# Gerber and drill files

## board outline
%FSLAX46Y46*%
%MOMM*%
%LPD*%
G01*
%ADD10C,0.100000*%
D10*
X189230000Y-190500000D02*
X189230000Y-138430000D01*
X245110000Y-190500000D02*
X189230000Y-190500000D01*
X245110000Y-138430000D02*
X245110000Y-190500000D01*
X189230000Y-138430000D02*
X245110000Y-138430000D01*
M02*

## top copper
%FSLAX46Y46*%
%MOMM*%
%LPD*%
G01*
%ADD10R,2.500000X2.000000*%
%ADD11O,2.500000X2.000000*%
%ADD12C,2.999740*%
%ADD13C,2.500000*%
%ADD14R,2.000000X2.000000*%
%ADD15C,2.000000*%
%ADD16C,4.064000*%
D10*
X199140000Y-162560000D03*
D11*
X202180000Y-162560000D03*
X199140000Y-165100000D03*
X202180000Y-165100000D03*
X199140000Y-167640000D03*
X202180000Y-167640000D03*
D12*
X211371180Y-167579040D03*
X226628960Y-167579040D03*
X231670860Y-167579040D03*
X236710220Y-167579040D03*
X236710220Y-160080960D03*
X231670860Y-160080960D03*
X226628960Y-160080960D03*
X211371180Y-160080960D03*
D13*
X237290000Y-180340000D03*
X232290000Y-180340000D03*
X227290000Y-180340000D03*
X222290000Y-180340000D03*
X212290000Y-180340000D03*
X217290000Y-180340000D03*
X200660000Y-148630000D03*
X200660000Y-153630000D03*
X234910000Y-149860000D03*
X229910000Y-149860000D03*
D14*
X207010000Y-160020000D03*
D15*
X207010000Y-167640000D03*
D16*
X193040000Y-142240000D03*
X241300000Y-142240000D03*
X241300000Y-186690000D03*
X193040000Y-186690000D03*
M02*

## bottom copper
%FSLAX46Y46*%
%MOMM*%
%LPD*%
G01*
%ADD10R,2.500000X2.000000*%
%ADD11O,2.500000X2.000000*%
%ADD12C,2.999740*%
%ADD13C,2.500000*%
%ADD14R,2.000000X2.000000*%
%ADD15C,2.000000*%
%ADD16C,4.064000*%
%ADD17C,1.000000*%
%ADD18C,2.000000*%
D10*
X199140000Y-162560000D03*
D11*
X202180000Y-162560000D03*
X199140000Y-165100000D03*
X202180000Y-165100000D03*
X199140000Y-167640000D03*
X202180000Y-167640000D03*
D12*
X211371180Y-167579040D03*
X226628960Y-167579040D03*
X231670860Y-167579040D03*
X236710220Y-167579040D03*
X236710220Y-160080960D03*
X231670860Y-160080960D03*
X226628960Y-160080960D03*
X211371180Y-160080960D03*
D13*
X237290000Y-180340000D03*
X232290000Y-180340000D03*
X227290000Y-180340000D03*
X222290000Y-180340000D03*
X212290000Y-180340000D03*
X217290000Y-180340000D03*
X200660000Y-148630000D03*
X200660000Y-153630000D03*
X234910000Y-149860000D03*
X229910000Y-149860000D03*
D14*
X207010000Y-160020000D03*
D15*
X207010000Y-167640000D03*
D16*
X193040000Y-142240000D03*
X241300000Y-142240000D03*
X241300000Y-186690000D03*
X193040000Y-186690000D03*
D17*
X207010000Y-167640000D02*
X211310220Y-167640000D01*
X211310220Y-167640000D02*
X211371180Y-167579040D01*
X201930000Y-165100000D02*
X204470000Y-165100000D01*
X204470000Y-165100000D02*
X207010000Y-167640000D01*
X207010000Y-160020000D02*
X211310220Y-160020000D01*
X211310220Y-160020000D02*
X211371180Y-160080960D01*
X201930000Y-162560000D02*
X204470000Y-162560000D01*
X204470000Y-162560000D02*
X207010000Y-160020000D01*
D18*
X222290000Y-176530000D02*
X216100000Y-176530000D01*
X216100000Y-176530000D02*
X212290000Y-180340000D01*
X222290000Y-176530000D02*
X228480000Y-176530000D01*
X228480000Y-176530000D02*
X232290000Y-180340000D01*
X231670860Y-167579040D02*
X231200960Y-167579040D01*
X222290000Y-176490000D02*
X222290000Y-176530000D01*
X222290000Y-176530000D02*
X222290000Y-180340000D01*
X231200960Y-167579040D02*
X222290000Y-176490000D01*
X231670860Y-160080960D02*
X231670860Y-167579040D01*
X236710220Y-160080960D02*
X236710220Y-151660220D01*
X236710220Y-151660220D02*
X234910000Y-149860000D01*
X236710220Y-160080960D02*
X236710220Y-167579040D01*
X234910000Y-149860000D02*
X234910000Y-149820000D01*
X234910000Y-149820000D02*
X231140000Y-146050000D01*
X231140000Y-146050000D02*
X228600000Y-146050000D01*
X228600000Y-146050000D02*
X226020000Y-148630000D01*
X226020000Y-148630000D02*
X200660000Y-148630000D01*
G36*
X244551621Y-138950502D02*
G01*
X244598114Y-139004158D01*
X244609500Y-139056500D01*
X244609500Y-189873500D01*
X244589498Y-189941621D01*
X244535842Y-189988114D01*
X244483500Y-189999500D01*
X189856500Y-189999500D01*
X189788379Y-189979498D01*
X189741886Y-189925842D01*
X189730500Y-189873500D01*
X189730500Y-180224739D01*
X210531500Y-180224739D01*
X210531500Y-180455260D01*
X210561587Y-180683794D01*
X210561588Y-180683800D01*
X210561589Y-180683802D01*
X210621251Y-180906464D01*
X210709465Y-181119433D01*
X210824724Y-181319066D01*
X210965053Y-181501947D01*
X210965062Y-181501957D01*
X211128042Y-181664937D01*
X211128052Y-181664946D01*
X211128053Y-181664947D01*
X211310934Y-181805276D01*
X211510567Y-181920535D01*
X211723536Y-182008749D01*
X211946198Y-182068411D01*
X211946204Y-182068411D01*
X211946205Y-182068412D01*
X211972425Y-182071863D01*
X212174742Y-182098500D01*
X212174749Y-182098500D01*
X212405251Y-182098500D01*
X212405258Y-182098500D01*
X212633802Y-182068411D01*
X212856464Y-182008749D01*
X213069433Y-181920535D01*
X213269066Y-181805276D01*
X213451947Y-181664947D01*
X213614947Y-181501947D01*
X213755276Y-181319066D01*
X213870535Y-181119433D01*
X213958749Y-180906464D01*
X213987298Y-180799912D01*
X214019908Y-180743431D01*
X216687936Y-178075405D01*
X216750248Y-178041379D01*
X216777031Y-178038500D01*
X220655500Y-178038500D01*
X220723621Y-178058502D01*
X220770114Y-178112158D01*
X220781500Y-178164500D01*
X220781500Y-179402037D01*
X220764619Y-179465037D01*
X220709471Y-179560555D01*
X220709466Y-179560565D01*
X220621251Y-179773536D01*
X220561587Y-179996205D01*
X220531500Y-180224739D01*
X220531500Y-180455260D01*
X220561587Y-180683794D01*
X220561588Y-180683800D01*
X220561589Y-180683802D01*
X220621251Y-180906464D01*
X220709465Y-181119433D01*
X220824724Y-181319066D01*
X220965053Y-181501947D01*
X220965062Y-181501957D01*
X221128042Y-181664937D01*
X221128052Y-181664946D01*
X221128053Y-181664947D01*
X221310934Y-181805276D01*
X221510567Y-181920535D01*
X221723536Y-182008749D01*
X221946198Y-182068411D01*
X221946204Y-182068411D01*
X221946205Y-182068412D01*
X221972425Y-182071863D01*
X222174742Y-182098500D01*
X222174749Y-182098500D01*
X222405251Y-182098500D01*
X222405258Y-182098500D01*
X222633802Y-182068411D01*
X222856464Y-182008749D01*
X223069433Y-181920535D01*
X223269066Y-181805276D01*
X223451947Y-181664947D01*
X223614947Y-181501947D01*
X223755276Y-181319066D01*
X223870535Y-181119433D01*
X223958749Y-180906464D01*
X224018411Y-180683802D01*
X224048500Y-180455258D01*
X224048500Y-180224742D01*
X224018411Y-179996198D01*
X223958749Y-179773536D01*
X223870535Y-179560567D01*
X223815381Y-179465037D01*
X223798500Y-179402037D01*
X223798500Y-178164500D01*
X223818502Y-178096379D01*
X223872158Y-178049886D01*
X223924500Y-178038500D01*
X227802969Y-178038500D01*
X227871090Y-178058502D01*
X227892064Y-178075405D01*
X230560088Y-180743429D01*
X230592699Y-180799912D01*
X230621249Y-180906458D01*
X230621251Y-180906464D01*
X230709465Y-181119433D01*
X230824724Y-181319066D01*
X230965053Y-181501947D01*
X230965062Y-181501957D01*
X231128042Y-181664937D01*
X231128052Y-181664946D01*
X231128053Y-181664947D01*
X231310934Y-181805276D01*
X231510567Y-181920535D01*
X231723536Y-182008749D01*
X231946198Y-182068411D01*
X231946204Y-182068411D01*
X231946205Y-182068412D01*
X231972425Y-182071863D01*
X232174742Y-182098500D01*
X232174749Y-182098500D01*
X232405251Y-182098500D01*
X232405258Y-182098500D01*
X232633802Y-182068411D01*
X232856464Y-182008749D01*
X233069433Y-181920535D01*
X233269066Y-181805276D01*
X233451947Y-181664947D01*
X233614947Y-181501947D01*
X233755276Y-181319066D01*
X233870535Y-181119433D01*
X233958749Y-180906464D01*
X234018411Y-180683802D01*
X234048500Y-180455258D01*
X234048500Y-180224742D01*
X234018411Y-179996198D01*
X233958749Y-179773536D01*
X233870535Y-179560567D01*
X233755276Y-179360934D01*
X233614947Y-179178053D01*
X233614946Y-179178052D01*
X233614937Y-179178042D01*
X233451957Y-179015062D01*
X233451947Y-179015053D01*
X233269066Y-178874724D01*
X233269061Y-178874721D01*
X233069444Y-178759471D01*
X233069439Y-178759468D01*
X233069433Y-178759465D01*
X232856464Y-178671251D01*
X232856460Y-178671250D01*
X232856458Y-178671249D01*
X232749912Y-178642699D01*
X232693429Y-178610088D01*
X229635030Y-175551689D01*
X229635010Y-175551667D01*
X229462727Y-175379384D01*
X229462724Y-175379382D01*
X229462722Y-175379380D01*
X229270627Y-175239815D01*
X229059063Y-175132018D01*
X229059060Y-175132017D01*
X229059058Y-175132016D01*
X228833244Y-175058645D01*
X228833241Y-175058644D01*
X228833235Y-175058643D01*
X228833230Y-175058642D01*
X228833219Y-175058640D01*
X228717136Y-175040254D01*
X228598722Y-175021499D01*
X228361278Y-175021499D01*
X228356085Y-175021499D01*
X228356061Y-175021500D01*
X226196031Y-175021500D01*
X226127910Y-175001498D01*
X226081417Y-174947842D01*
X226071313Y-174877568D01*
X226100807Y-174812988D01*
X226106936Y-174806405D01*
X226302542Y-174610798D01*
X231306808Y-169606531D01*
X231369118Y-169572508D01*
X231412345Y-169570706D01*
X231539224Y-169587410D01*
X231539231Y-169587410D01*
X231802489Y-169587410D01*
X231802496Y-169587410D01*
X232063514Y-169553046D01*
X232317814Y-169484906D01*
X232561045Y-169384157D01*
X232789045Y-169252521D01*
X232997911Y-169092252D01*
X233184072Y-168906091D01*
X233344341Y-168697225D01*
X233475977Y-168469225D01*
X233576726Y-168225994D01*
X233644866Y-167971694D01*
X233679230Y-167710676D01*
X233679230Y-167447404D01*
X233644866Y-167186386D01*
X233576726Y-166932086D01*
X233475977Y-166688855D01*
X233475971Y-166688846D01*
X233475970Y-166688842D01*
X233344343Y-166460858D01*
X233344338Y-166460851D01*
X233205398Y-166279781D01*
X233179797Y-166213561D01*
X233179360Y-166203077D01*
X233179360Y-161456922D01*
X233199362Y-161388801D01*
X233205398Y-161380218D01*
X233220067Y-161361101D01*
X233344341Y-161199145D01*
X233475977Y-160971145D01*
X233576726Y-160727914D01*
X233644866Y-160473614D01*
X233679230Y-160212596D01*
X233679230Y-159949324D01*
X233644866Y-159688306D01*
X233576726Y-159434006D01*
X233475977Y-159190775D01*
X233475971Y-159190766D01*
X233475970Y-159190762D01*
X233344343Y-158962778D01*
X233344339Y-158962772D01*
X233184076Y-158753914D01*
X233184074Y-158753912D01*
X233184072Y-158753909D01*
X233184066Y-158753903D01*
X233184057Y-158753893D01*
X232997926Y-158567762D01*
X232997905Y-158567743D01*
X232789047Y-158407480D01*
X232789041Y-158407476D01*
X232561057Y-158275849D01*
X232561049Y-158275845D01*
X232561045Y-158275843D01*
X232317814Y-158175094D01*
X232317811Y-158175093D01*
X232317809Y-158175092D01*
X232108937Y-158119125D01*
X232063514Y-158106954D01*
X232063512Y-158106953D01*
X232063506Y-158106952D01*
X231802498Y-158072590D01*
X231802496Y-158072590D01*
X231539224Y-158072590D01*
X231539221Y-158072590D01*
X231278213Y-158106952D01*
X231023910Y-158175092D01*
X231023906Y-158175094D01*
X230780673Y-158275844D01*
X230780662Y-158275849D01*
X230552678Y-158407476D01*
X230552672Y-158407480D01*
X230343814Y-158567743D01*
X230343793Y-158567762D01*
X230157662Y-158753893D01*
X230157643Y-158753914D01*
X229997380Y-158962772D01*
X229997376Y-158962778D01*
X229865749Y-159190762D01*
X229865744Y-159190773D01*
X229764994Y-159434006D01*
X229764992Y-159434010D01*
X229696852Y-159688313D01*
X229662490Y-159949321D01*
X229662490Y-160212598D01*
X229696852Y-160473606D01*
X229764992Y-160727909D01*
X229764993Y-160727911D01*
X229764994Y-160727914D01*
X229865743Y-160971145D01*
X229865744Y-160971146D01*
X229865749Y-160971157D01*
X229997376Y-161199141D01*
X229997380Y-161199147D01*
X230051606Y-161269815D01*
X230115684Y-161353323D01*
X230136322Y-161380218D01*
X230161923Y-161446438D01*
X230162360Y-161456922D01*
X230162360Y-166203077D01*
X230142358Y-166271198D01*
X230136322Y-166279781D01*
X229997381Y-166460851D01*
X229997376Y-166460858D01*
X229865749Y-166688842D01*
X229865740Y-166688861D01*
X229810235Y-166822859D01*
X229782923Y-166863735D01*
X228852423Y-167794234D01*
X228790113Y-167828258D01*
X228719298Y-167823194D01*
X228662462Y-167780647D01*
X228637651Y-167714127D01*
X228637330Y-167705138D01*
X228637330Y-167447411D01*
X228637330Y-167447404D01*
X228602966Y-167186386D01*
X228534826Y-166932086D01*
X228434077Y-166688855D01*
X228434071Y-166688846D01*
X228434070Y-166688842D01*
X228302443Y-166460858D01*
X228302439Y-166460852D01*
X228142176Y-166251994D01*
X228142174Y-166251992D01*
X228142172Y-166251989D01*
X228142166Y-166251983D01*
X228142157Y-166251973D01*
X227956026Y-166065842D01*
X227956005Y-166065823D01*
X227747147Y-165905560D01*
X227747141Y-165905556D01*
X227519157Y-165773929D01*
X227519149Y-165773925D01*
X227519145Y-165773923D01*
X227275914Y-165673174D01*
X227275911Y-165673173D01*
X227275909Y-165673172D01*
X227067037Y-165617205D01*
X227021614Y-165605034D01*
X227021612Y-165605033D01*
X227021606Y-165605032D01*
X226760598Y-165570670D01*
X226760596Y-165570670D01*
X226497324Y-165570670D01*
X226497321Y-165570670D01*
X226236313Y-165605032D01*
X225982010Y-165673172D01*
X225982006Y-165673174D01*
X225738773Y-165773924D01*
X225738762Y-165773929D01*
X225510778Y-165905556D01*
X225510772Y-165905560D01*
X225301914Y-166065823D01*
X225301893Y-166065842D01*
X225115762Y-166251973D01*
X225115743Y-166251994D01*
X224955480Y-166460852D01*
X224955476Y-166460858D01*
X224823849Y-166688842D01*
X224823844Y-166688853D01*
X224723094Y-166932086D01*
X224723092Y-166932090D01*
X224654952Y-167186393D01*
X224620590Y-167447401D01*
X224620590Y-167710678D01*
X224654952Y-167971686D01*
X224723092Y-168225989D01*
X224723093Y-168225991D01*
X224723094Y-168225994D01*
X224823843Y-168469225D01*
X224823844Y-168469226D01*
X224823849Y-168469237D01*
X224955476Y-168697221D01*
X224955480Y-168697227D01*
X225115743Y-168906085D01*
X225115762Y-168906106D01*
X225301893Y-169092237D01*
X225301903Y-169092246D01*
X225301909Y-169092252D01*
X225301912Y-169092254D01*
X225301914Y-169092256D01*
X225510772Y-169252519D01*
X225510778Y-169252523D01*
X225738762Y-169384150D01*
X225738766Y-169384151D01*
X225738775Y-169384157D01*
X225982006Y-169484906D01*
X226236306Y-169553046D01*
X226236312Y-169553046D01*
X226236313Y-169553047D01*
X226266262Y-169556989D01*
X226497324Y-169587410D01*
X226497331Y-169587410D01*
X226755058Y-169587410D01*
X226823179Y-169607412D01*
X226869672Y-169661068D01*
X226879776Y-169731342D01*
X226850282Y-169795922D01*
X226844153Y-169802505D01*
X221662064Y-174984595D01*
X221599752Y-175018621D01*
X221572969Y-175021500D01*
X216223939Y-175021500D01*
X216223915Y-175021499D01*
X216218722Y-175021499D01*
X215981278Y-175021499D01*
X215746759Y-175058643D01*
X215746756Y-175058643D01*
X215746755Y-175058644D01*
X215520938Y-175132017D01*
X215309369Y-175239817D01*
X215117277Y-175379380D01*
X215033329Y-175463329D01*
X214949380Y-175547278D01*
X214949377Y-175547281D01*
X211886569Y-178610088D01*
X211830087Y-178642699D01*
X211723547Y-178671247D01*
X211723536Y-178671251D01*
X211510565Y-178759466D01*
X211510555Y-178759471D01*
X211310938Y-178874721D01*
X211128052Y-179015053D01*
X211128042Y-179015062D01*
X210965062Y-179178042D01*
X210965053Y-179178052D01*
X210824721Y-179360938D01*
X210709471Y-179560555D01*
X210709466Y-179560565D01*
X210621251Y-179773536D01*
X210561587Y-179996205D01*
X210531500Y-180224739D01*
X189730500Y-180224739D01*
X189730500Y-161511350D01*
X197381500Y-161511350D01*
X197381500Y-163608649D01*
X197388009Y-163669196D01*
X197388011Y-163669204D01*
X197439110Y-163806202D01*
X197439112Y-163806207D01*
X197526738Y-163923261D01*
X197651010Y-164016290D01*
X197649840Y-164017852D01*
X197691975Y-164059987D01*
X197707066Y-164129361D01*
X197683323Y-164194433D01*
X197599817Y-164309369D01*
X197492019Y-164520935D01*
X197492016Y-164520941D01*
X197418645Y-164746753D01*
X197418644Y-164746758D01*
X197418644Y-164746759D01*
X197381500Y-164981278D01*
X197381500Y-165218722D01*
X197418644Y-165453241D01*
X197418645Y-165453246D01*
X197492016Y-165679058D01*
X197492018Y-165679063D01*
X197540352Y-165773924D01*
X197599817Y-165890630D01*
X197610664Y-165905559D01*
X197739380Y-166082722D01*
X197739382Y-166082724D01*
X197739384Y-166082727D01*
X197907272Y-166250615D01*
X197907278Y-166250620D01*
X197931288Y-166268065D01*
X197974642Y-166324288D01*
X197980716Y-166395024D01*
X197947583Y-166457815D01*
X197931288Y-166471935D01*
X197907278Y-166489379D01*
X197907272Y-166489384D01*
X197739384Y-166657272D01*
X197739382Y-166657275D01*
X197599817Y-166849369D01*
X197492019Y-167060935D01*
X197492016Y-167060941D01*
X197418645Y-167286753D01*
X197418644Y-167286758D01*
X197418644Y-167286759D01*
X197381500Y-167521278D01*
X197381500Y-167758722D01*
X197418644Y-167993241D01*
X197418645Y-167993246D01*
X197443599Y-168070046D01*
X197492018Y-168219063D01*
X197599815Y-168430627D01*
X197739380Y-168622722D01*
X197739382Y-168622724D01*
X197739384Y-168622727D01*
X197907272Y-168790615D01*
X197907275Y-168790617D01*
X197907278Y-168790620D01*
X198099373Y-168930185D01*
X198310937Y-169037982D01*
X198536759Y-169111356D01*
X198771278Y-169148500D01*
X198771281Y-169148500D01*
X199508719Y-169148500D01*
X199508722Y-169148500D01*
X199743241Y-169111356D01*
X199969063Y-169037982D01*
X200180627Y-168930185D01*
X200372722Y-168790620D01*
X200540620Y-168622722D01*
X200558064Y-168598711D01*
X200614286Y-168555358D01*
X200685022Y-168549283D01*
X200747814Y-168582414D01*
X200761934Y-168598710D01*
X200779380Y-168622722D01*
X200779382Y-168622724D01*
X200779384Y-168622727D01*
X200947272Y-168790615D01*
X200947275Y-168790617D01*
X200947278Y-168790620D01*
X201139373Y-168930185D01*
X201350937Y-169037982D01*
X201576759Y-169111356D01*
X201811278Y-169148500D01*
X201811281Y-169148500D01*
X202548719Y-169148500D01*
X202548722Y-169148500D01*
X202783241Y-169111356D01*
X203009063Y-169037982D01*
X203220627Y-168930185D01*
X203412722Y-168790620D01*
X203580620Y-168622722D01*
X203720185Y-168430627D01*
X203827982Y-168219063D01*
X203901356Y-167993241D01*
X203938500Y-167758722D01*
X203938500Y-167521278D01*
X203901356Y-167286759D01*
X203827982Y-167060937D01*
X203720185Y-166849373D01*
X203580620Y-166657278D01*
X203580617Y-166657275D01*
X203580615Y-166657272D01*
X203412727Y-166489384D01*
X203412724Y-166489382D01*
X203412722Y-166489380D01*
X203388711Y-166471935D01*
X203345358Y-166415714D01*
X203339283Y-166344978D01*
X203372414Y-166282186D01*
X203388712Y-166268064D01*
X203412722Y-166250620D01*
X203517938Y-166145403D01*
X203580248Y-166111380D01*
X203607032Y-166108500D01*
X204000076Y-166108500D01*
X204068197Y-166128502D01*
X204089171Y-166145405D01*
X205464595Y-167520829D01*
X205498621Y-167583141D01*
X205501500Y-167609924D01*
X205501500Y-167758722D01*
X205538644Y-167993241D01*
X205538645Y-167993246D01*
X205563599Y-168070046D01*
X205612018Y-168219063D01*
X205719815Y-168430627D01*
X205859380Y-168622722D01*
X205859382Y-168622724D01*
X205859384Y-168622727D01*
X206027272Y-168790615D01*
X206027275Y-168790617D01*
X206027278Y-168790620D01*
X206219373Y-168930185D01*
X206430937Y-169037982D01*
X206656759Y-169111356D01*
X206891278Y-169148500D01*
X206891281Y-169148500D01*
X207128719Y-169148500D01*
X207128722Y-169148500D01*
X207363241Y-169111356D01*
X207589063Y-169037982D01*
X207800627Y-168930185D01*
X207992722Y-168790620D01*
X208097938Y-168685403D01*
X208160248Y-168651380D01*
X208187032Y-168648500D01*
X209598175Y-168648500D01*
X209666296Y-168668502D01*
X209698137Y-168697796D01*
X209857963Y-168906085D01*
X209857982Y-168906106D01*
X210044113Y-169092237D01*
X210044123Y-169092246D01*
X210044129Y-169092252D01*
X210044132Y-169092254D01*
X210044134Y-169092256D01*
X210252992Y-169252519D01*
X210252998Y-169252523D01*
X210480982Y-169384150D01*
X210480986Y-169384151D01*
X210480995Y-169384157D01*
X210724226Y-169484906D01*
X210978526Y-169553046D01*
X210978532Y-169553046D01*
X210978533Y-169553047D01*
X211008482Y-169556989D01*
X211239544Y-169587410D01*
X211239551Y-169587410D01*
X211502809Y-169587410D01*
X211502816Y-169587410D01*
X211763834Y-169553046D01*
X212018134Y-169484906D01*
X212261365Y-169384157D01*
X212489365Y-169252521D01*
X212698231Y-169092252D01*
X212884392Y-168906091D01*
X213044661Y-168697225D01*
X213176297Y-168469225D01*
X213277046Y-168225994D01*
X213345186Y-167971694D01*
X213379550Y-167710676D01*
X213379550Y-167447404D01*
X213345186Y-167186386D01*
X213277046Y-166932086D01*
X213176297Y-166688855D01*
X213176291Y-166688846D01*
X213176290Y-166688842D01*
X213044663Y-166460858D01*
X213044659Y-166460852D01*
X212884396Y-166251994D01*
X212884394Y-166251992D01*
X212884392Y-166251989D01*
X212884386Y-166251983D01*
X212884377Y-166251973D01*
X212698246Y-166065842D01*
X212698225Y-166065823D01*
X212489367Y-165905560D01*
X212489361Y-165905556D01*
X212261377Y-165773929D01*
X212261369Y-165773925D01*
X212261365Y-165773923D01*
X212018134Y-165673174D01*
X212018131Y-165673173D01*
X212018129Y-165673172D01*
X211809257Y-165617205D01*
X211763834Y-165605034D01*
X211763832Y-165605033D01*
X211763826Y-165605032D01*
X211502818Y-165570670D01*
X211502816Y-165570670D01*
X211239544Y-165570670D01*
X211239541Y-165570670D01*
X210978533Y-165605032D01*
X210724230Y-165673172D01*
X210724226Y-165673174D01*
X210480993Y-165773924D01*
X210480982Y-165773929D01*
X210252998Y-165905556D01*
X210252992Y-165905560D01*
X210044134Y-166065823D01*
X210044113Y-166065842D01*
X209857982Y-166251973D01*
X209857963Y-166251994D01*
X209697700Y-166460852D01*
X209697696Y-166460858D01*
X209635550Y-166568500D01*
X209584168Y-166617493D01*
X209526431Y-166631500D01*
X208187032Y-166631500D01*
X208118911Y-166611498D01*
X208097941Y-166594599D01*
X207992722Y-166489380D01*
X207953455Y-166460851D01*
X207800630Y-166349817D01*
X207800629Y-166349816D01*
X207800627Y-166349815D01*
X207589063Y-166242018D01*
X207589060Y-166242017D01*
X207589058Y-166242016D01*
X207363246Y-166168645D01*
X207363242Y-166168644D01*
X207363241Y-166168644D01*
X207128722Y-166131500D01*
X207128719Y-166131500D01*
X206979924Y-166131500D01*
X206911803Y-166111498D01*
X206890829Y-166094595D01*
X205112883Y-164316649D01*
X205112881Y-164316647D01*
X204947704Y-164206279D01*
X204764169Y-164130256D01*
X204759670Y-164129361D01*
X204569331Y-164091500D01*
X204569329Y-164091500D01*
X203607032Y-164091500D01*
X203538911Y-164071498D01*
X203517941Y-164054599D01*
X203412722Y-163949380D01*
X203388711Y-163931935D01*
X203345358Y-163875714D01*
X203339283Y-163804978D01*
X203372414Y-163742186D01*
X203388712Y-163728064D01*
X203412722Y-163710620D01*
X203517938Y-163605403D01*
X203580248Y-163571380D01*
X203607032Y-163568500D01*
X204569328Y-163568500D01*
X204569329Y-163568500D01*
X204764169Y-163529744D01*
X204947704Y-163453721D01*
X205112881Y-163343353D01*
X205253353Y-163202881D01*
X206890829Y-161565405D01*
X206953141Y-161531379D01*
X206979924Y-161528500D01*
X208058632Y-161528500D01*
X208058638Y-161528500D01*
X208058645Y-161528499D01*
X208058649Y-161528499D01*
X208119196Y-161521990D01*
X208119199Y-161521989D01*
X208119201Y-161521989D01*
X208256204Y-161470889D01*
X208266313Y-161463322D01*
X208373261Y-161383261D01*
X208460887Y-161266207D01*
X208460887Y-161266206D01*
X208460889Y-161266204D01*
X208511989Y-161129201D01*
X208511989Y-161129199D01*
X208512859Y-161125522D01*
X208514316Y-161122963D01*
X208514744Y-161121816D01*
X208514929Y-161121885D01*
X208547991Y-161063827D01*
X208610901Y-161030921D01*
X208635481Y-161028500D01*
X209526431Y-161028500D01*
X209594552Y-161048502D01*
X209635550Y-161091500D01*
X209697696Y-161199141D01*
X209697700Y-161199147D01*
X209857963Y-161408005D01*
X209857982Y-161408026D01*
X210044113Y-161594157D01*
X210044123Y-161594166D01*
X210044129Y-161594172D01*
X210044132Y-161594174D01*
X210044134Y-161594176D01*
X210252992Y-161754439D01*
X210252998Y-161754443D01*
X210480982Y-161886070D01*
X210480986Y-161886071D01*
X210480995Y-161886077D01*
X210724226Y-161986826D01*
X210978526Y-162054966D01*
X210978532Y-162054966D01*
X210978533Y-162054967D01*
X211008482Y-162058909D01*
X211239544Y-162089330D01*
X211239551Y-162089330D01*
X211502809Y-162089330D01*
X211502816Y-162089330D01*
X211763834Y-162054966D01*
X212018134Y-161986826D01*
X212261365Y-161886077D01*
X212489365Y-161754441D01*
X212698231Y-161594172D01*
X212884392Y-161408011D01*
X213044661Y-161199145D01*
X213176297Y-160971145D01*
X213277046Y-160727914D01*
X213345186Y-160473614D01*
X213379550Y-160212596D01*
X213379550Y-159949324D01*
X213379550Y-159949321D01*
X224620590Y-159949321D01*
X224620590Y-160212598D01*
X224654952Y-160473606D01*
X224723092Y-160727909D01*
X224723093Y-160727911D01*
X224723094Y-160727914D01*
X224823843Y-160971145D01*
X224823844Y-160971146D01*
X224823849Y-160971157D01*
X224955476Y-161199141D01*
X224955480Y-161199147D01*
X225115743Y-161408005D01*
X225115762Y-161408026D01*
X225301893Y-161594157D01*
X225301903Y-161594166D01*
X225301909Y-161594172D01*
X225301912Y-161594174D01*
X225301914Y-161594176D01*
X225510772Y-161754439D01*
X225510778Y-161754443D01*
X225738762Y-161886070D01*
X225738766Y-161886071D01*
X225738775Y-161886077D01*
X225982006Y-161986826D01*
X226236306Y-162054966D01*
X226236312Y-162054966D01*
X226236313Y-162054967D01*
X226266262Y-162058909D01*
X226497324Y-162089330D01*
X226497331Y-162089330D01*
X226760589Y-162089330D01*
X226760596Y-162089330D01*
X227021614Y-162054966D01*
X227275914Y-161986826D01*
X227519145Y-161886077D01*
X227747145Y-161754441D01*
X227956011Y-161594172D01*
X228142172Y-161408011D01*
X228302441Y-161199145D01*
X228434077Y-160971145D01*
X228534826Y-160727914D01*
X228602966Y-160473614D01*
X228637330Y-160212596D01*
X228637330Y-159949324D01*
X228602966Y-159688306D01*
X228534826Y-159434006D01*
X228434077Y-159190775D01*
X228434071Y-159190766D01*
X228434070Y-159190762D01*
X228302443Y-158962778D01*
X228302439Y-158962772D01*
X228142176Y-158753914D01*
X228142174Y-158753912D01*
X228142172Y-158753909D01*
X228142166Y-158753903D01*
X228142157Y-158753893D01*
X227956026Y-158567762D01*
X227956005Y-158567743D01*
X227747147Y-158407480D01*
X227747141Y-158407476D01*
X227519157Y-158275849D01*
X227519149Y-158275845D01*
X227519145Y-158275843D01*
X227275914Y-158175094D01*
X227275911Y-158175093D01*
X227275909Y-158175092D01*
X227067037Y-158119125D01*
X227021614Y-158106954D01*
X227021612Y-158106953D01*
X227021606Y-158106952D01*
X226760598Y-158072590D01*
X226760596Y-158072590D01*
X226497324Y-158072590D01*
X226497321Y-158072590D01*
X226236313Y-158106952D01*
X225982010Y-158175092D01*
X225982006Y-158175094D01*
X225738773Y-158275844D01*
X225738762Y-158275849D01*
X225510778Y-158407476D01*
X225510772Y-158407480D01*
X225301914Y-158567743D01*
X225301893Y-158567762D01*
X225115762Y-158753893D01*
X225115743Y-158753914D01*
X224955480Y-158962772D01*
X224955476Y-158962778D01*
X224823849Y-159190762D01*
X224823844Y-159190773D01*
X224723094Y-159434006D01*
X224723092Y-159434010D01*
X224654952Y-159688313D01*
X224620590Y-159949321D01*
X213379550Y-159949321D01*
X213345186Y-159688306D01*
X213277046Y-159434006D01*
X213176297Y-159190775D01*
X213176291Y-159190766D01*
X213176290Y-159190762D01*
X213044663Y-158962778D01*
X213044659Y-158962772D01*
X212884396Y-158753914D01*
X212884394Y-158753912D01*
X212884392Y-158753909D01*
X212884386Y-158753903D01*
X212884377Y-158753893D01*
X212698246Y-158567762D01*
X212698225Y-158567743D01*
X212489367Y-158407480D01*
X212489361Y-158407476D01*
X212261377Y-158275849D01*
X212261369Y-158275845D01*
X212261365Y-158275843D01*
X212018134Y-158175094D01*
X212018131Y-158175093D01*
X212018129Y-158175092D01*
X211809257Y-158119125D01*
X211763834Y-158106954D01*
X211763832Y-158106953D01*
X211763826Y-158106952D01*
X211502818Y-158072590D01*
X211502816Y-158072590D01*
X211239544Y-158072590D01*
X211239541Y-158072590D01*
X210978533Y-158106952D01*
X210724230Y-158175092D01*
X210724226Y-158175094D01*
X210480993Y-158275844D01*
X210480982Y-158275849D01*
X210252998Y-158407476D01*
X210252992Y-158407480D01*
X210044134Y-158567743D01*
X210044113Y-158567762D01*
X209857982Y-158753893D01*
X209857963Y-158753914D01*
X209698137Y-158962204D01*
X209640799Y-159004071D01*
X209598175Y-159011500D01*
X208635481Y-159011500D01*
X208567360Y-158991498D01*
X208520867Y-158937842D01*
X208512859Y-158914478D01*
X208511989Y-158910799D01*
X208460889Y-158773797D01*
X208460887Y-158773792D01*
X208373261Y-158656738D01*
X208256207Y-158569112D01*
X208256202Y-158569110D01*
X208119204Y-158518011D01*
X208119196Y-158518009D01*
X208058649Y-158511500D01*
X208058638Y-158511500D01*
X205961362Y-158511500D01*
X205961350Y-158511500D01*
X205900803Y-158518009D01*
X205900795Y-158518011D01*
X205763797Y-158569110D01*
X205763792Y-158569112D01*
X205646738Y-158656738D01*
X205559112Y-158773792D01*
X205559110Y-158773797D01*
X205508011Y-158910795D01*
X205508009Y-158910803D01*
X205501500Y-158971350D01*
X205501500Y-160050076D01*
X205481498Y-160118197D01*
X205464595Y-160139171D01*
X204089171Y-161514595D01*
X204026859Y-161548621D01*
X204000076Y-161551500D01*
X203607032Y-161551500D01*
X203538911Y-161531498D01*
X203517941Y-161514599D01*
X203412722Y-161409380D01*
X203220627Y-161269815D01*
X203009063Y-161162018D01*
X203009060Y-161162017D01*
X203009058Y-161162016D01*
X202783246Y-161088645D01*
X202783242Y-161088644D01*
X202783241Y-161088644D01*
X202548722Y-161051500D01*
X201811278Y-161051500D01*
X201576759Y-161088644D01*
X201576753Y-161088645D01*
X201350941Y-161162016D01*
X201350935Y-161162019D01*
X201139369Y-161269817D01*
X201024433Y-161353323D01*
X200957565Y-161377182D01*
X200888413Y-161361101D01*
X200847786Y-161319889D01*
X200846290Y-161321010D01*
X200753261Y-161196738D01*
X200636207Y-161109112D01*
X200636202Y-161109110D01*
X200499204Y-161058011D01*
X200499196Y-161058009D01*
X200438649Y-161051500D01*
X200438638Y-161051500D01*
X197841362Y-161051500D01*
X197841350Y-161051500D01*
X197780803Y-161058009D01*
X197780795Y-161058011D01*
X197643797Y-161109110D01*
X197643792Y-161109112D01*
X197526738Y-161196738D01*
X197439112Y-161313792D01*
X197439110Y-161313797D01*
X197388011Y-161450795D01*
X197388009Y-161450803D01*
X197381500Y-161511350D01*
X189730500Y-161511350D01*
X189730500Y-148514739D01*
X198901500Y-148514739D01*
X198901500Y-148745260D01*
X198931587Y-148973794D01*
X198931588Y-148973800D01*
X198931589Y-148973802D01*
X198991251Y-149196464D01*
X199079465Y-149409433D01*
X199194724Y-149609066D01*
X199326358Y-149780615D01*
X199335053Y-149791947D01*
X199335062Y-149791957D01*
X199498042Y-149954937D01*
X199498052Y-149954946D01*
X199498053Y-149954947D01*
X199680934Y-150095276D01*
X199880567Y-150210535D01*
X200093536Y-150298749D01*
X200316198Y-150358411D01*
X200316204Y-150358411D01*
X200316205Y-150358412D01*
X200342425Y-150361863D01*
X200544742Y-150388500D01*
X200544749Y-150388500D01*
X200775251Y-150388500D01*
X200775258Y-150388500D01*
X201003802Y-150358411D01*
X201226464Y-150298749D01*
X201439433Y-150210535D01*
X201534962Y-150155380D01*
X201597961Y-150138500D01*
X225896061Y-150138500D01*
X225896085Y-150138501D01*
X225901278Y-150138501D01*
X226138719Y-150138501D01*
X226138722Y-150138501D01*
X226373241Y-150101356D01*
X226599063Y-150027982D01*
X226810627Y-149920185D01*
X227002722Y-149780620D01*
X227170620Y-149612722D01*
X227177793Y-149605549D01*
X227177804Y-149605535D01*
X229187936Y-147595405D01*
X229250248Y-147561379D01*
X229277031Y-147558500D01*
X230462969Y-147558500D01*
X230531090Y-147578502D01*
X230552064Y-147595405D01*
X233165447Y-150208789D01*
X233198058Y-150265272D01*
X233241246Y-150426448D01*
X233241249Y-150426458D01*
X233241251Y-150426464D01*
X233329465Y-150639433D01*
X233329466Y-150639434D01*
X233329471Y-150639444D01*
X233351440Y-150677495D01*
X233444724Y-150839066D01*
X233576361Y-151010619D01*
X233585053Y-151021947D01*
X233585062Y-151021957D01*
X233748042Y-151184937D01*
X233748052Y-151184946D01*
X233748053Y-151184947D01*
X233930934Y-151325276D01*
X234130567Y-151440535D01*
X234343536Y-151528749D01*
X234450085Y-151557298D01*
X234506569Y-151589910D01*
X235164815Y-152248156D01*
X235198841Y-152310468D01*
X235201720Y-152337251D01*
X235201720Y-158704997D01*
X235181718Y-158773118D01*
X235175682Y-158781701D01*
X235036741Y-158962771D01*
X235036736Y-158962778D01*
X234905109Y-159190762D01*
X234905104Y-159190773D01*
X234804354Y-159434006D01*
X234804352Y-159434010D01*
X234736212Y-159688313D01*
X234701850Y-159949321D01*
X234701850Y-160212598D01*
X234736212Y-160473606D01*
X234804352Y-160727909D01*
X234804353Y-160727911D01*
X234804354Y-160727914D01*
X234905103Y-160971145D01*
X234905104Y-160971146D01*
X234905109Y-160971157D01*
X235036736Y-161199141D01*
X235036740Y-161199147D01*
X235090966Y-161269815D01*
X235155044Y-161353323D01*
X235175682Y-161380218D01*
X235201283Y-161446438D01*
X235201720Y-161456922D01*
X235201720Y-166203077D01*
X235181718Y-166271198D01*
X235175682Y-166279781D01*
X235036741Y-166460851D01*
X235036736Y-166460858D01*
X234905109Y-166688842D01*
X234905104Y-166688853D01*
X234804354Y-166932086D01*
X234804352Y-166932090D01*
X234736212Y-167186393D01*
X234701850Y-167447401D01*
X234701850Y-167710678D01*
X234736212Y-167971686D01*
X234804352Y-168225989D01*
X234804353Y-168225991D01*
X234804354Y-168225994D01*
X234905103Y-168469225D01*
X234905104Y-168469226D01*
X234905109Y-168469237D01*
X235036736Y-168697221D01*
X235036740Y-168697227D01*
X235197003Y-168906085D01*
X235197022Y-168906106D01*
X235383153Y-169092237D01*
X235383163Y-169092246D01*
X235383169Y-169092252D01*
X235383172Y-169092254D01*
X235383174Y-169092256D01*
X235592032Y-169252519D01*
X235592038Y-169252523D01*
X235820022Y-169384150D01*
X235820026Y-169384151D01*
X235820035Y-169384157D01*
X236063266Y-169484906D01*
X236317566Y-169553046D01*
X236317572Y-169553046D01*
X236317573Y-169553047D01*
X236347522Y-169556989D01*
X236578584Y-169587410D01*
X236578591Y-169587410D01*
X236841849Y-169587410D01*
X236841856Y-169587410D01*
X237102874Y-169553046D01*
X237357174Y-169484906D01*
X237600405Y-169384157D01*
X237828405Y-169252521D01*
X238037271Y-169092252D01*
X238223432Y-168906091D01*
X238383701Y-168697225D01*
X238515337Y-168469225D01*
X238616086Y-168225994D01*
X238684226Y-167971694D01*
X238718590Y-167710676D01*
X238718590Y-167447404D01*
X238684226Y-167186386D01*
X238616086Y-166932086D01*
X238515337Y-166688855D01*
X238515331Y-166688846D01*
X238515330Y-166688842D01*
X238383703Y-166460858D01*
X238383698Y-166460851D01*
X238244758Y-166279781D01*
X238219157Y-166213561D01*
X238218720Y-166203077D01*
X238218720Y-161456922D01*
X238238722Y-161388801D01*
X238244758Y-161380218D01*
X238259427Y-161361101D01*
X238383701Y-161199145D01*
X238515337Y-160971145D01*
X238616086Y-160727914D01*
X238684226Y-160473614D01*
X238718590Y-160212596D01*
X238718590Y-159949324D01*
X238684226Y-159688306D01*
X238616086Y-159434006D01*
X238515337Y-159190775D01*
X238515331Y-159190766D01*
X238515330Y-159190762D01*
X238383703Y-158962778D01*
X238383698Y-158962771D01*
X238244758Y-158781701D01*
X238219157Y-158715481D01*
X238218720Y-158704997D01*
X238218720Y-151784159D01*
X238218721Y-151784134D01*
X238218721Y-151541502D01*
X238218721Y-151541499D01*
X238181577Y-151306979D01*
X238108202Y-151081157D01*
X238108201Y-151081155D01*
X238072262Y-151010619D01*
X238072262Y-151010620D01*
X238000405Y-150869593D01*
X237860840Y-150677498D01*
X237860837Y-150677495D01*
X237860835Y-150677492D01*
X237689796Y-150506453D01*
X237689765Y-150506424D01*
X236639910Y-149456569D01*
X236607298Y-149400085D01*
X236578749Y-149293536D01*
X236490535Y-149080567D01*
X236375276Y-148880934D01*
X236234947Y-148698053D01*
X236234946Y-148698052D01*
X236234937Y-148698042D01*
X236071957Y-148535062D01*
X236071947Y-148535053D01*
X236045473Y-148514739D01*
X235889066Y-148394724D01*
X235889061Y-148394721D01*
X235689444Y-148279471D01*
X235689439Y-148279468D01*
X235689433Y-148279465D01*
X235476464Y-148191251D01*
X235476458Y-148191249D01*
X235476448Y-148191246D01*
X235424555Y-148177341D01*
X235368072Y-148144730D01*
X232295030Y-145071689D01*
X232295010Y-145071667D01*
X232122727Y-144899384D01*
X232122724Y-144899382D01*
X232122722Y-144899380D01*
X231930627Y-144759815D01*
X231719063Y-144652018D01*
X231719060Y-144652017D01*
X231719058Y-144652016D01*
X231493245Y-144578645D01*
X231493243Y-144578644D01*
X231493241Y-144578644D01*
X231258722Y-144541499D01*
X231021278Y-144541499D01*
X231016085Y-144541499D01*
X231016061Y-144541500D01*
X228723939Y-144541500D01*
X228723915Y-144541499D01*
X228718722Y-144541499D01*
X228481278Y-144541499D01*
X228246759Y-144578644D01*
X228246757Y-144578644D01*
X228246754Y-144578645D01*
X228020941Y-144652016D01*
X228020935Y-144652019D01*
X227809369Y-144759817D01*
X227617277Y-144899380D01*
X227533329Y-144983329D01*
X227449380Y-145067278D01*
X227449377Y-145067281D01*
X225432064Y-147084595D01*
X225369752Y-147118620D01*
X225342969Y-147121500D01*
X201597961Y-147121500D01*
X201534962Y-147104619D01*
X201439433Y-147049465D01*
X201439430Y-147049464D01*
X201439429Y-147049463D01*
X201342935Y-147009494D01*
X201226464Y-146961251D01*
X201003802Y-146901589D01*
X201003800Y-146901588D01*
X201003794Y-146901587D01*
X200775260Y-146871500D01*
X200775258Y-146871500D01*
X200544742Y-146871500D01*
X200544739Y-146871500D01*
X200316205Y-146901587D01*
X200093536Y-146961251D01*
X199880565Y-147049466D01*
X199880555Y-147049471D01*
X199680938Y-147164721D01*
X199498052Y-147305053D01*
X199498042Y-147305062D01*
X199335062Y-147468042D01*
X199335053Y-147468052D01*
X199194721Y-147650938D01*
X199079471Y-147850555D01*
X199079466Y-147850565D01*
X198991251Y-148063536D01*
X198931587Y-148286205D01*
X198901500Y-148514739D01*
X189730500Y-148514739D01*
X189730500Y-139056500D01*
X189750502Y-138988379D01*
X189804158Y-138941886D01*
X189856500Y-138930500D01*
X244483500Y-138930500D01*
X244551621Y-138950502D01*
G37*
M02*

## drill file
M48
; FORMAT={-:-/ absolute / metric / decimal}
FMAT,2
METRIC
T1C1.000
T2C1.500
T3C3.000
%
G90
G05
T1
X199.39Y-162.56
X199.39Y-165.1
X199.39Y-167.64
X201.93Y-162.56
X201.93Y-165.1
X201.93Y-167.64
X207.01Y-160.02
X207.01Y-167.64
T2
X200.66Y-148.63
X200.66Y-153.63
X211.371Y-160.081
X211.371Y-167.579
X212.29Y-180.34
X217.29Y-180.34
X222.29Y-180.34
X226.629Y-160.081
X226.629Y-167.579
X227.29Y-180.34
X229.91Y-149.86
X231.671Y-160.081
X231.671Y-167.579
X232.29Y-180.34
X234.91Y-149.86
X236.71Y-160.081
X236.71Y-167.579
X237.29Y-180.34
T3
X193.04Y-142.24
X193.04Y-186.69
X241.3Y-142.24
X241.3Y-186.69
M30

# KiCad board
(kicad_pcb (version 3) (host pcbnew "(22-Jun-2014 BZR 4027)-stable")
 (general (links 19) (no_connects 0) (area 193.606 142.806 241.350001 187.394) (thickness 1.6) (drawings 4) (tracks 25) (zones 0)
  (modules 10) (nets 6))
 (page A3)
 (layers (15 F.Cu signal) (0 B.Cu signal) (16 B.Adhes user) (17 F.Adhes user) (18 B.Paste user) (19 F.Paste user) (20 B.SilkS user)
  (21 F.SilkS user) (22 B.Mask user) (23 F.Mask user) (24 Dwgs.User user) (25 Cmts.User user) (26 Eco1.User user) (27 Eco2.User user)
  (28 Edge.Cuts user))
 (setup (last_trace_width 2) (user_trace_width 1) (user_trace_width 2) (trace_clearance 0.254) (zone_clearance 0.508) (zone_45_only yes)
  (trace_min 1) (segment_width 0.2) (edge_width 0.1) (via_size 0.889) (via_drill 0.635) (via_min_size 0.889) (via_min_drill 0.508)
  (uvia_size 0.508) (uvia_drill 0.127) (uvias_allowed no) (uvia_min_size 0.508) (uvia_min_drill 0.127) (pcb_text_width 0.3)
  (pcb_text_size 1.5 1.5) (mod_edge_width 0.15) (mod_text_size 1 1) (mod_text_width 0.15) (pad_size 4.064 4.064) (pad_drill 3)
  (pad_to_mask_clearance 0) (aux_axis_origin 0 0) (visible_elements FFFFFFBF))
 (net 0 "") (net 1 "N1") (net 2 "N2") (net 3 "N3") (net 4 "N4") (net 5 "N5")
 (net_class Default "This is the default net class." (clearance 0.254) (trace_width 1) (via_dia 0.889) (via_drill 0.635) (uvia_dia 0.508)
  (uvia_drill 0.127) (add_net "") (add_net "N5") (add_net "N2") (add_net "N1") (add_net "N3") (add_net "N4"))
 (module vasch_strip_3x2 (layer F.Cu) (at 200.66 165.1 270)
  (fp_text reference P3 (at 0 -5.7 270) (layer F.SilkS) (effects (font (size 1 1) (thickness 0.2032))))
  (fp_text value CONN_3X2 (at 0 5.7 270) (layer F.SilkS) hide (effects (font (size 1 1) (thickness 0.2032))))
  (pad 1 thru_hole rect (at -2.54 1.27 270) (size 2 2.5) (drill 1 (offset 0 0.25)) (layers *.Cu *.Mask F.SilkS))
  (pad 2 thru_hole oval (at -2.54 -1.27 270) (size 2 2.5) (drill 1 (offset 0 -0.25)) (layers *.Cu *.Mask F.SilkS) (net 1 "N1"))
  (pad 3 thru_hole oval (at 0 1.27 270) (size 2 2.5) (drill 1 (offset 0 0.25)) (layers *.Cu *.Mask F.SilkS))
  (pad 4 thru_hole oval (at 0 -1.27 270) (size 2 2.5) (drill 1 (offset 0 -0.25)) (layers *.Cu *.Mask F.SilkS) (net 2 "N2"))
  (pad 5 thru_hole oval (at 2.54 1.27 270) (size 2 2.5) (drill 1 (offset 0 0.25)) (layers *.Cu *.Mask F.SilkS))
  (pad 6 thru_hole oval (at 2.54 -1.27 270) (size 2 2.5) (drill 1 (offset 0 -0.25)) (layers *.Cu *.Mask F.SilkS)))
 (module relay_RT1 (layer F.Cu) (at 223.52 163.83)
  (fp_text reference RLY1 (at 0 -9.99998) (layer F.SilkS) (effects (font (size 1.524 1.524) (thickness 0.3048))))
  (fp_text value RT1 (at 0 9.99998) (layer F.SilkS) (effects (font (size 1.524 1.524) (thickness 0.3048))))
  (pad 1 thru_hole circle (at -12.14882 3.74904) (size 2.99974 2.99974) (drill 1.5) (layers *.Cu *.Mask F.SilkS) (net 2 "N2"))
  (pad 12 thru_hole circle (at 3.10896 3.74904) (size 2.99974 2.99974) (drill 1.5) (layers *.Cu *.Mask F.SilkS))
  (pad 11 thru_hole circle (at 8.15086 3.74904) (size 2.99974 2.99974) (drill 1.5) (layers *.Cu *.Mask F.SilkS) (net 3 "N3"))
  (pad 14 thru_hole circle (at 13.19022 3.74904) (size 2.99974 2.99974) (drill 1.5) (layers *.Cu *.Mask F.SilkS) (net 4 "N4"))
  (pad 14 thru_hole circle (at 13.19022 -3.74904) (size 2.99974 2.99974) (drill 1.5) (layers *.Cu *.Mask F.SilkS) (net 4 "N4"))
  (pad 11 thru_hole circle (at 8.15086 -3.74904) (size 2.99974 2.99974) (drill 1.5) (layers *.Cu *.Mask F.SilkS) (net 3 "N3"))
  (pad 12 thru_hole circle (at 3.10896 -3.74904) (size 2.99974 2.99974) (drill 1.5) (layers *.Cu *.Mask F.SilkS))
  (pad 2 thru_hole circle (at -12.14882 -3.74904) (size 2.99974 2.99974) (drill 1.5) (layers *.Cu *.Mask F.SilkS) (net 1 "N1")))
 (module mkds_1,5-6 (layer F.Cu) (at 224.79 180.34)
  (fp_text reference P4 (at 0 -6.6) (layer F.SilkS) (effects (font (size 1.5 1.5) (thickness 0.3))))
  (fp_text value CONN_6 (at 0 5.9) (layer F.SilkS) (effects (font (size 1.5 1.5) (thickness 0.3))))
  (pad 6 thru_hole circle (at 12.5 0) (size 2.5 2.5) (drill 1.5) (layers *.Cu *.Mask F.SilkS) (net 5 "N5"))
  (pad 5 thru_hole circle (at 7.5 0) (size 2.5 2.5) (drill 1.5) (layers *.Cu *.Mask F.SilkS) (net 3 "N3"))
  (pad 4 thru_hole circle (at 2.5 0) (size 2.5 2.5) (drill 1.5) (layers *.Cu *.Mask F.SilkS) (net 5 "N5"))
  (pad 3 thru_hole circle (at -2.5 0) (size 2.5 2.5) (drill 1.5) (layers *.Cu *.Mask F.SilkS) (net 3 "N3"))
  (pad 1 thru_hole circle (at -12.5 0) (size 2.5 2.5) (drill 1.5) (layers *.Cu *.Mask F.SilkS) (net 3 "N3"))
  (pad 2 thru_hole circle (at -7.5 0) (size 2.5 2.5) (drill 1.5) (layers *.Cu *.Mask F.SilkS) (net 5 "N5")))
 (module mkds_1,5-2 (layer F.Cu) (at 200.66 151.13 270)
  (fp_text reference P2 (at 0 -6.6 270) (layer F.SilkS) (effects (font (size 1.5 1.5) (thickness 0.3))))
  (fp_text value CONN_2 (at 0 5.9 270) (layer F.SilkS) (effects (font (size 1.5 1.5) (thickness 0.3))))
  (pad 1 thru_hole circle (at -2.5 0 270) (size 2.5 2.5) (drill 1.5) (layers *.Cu *.Mask F.SilkS) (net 4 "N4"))
  (pad 2 thru_hole circle (at 2.5 0 270) (size 2.5 2.5) (drill 1.5) (layers *.Cu *.Mask F.SilkS) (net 5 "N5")))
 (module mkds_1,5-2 (layer F.Cu) (at 232.41 149.86 180)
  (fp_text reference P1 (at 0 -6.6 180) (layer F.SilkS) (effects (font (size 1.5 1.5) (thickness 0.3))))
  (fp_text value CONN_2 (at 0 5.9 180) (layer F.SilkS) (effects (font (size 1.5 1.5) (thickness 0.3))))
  (pad 1 thru_hole circle (at -2.5 0 180) (size 2.5 2.5) (drill 1.5) (layers *.Cu *.Mask F.SilkS) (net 4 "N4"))
  (pad 2 thru_hole circle (at 2.5 0 180) (size 2.5 2.5) (drill 1.5) (layers *.Cu *.Mask F.SilkS) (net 5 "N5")))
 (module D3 (layer F.Cu) (at 207.01 163.83 90)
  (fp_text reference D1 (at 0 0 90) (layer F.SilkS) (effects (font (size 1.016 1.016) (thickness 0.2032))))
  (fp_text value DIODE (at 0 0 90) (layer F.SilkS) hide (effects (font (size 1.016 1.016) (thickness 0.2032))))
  (pad 2 thru_hole rect (at 3.81 0 90) (size 2 2) (drill 1) (layers *.Cu *.Mask F.SilkS) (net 1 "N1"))
  (pad 1 thru_hole circle (at -3.81 0 90) (size 2 2) (drill 1) (layers *.Cu *.Mask F.SilkS) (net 2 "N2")))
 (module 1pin (layer F.Cu) (at 193.04 142.24)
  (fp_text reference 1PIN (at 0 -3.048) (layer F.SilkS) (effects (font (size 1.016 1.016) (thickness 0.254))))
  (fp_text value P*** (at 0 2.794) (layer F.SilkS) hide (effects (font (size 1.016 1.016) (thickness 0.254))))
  (pad 1 thru_hole circle (at 0 0) (size 4.064 4.064) (drill 3) (layers *.Cu *.Mask F.SilkS) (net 5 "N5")))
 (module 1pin (layer F.Cu) (at 241.3 142.24)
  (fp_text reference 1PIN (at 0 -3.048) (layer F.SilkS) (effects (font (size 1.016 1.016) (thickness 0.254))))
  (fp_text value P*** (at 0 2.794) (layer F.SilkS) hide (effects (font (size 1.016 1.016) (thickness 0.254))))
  (pad 1 thru_hole circle (at 0 0) (size 4.064 4.064) (drill 3) (layers *.Cu *.Mask F.SilkS) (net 5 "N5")))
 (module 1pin (layer F.Cu) (at 241.3 186.69)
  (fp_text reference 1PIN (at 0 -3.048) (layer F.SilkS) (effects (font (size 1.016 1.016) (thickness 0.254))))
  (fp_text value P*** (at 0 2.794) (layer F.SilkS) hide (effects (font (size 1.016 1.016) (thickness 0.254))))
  (pad 1 thru_hole circle (at 0 0) (size 4.064 4.064) (drill 3) (layers *.Cu *.Mask F.SilkS) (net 5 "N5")))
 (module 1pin (layer F.Cu) (at 193.04 186.69)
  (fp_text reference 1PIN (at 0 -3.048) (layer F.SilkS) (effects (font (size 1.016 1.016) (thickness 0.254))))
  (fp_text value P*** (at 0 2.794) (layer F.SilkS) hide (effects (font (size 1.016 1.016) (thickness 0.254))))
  (pad 1 thru_hole circle (at 0 0) (size 4.064 4.064) (drill 3) (layers *.Cu *.Mask F.SilkS) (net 5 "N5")))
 (gr_line (start 189.23 190.5) (end 189.23 138.43) (angle 90) (layer Edge.Cuts) (width 0.1))
 (gr_line (start 245.11 190.5) (end 189.23 190.5) (angle 90) (layer Edge.Cuts) (width 0.1))
 (gr_line (start 245.11 138.43) (end 245.11 190.5) (angle 90) (layer Edge.Cuts) (width 0.1))
 (gr_line (start 189.23 138.43) (end 245.11 138.43) (angle 90) (layer Edge.Cuts) (width 0.1))
 (segment (start 207.01 167.64) (end 211.31022 167.64) (width 1) (layer B.Cu) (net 2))
 (segment (start 211.31022 167.64) (end 211.37118 167.57904) (width 1) (layer B.Cu) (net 2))
 (segment (start 201.93 165.1) (end 204.47 165.1) (width 1) (layer B.Cu) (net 2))
 (segment (start 204.47 165.1) (end 207.01 167.64) (width 1) (layer B.Cu) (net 2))
 (segment (start 207.01 160.02) (end 211.31022 160.02) (width 1) (layer B.Cu) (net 1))
 (segment (start 211.31022 160.02) (end 211.37118 160.08096) (width 1) (layer B.Cu) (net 1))
 (segment (start 201.93 162.56) (end 204.47 162.56) (width 1) (layer B.Cu) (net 1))
 (segment (start 204.47 162.56) (end 207.01 160.02) (width 1) (layer B.Cu) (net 1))
 (segment (start 222.29 176.53) (end 216.1 176.53) (width 2) (layer B.Cu) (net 3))
 (segment (start 216.1 176.53) (end 212.29 180.34) (width 2) (layer B.Cu) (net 3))
 (segment (start 222.29 176.53) (end 228.48 176.53) (width 2) (layer B.Cu) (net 3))
 (segment (start 228.48 176.53) (end 232.29 180.34) (width 2) (layer B.Cu) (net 3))
 (segment (start 231.67086 167.57904) (end 231.20096 167.57904) (width 2) (layer B.Cu) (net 3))
 (segment (start 222.29 176.49) (end 222.29 176.53) (width 2) (layer B.Cu) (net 3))
 (segment (start 222.29 176.53) (end 222.29 180.34) (width 2) (layer B.Cu) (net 3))
 (segment (start 231.20096 167.57904) (end 222.29 176.49) (width 2) (layer B.Cu) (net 3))
 (segment (start 231.67086 160.08096) (end 231.67086 167.57904) (width 2) (layer B.Cu) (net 3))
 (segment (start 236.71022 160.08096) (end 236.71022 151.66022) (width 2) (layer B.Cu) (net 4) (status 400000))
 (segment (start 236.71022 151.66022) (end 234.91 149.86) (width 2) (layer B.Cu) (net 4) (status 800000))
 (segment (start 236.71022 160.08096) (end 236.71022 167.57904) (width 2) (layer B.Cu) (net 4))
 (segment (start 234.91 149.86) (end 234.91 149.82) (width 2) (layer B.Cu) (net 4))
 (segment (start 234.91 149.82) (end 231.14 146.05) (width 2) (layer B.Cu) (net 4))
 (segment (start 231.14 146.05) (end 228.6 146.05) (width 2) (layer B.Cu) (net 4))
 (segment (start 228.6 146.05) (end 226.02 148.63) (width 2) (layer B.Cu) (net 4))
 (segment (start 226.02 148.63) (end 200.66 148.63) (width 2) (layer B.Cu) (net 4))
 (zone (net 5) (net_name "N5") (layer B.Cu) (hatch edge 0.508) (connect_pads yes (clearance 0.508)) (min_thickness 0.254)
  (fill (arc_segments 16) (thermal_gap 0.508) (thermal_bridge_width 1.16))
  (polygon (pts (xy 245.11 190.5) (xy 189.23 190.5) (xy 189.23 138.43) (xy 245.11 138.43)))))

